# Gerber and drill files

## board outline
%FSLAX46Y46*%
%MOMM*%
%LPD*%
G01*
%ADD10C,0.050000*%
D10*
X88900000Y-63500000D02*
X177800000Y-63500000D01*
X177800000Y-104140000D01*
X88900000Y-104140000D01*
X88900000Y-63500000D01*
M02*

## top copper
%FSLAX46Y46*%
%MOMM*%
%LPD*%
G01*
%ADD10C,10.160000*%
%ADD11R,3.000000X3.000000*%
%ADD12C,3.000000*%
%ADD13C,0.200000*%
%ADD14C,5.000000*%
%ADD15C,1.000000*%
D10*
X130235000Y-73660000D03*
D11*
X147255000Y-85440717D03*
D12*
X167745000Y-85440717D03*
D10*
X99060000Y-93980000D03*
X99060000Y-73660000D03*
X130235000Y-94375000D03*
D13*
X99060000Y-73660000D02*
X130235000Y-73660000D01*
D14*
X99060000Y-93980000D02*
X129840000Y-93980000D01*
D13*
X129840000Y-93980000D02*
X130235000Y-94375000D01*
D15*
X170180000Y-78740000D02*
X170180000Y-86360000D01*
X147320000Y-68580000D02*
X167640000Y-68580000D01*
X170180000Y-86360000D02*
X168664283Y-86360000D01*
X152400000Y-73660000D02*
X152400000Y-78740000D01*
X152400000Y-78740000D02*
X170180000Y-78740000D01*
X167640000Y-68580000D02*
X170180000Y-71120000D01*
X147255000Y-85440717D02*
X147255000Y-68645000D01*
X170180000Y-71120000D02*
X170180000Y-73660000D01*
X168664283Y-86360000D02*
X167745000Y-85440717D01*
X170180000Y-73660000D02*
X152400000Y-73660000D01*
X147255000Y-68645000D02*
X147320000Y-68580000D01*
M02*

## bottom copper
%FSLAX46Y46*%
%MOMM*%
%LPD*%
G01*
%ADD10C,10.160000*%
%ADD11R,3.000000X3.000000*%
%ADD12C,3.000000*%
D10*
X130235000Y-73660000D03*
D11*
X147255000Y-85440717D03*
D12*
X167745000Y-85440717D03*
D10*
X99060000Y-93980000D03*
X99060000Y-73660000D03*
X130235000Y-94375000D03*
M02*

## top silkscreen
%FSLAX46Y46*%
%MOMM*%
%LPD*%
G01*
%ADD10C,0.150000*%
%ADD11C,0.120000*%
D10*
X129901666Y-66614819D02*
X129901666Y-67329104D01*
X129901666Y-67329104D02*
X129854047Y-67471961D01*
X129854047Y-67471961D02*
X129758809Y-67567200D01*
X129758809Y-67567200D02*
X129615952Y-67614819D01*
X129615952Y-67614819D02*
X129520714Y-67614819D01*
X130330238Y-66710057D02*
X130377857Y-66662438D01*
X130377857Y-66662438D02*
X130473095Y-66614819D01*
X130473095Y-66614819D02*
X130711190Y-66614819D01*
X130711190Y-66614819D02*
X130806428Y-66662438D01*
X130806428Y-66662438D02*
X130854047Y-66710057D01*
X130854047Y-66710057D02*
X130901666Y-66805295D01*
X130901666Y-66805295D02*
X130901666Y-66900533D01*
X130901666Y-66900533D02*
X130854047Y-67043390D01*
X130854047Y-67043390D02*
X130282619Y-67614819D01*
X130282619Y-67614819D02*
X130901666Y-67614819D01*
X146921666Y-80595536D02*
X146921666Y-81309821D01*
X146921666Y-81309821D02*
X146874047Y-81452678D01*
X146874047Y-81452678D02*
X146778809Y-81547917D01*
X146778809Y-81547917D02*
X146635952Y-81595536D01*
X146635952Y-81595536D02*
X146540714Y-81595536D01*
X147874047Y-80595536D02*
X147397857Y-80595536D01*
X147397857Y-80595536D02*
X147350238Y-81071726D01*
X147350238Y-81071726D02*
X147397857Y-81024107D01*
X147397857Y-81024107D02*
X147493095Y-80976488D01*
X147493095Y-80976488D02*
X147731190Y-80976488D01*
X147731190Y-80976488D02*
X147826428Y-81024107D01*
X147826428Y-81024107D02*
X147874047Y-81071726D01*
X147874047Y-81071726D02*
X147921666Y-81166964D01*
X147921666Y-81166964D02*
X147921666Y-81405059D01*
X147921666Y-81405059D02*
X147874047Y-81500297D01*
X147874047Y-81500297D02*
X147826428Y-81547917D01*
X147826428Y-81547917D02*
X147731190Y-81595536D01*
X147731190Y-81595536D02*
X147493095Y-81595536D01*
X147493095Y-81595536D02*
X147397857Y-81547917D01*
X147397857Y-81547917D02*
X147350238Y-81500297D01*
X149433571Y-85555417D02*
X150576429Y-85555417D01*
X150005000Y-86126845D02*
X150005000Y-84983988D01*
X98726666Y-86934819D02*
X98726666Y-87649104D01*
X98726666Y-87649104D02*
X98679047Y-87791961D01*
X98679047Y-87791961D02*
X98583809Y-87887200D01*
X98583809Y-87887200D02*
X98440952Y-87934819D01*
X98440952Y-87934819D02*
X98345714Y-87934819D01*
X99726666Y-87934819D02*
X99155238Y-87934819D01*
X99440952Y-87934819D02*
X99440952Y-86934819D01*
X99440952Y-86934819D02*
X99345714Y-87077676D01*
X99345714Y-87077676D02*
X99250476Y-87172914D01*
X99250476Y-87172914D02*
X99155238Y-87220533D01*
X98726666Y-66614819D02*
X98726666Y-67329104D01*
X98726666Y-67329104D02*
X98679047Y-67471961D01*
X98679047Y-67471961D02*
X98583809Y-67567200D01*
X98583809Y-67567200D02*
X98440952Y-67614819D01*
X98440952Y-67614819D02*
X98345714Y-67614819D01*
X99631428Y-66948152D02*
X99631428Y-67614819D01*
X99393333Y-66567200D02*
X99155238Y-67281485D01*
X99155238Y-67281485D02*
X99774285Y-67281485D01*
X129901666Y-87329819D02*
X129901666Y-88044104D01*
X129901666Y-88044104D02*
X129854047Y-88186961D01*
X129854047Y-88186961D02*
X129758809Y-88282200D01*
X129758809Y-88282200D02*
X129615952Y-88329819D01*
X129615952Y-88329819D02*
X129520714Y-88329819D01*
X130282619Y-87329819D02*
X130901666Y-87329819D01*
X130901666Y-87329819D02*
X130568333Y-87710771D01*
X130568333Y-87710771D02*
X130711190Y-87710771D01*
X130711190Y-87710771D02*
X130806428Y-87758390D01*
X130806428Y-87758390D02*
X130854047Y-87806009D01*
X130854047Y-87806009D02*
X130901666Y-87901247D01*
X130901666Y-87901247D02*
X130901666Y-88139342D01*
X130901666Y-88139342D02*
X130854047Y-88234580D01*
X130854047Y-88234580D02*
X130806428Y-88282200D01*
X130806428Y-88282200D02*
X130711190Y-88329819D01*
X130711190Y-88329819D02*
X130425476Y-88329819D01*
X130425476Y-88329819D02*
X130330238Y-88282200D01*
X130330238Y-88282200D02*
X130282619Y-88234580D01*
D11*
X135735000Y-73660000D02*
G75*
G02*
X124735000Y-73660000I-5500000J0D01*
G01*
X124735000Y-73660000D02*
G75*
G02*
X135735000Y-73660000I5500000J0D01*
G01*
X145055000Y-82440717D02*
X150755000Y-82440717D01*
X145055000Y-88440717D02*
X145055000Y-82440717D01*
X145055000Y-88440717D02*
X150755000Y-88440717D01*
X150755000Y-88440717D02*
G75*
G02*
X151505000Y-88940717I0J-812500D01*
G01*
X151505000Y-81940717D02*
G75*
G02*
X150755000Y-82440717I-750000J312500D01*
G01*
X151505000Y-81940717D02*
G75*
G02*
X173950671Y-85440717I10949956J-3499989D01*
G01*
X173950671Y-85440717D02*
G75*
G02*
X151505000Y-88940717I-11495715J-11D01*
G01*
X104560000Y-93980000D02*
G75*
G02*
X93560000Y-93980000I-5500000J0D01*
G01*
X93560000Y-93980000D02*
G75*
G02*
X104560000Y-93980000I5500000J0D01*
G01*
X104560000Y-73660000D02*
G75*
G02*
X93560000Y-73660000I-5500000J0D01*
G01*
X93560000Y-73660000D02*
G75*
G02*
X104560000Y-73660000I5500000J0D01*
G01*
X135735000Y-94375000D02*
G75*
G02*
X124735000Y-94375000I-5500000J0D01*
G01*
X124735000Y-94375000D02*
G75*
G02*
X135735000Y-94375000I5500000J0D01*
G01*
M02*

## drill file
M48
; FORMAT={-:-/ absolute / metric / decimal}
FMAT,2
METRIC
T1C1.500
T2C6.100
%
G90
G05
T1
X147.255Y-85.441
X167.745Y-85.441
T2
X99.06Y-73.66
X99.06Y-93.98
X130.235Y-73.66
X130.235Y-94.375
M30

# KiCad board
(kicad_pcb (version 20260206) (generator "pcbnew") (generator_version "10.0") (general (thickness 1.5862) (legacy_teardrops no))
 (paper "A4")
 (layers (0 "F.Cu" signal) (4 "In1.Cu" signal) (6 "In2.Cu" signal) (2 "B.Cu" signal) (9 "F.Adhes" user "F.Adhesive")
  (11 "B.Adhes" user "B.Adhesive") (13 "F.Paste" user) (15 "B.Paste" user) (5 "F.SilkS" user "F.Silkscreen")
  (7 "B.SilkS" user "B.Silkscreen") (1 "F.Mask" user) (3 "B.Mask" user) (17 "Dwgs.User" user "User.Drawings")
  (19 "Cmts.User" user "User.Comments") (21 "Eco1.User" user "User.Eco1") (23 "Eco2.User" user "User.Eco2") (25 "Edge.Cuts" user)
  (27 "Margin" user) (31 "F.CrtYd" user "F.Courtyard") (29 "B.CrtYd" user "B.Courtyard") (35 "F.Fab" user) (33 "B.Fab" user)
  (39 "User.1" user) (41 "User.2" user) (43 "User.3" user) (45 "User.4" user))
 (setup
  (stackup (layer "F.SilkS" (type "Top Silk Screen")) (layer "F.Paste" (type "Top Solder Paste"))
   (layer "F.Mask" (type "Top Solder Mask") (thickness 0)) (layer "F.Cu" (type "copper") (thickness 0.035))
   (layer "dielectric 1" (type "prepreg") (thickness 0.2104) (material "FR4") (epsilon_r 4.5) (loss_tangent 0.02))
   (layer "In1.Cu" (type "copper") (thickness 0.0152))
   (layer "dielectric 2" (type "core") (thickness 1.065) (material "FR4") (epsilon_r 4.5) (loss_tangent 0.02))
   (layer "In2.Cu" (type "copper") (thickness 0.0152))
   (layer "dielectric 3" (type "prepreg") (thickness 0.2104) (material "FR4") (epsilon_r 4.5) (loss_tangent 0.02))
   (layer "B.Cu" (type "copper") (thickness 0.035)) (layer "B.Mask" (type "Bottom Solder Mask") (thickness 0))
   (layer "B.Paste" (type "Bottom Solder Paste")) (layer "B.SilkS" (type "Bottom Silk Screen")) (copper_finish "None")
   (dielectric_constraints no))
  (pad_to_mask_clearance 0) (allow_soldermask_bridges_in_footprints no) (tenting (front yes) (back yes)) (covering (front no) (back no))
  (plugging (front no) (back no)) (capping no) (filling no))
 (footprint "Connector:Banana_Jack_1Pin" (layer "F.Cu") (at 130.235 73.66)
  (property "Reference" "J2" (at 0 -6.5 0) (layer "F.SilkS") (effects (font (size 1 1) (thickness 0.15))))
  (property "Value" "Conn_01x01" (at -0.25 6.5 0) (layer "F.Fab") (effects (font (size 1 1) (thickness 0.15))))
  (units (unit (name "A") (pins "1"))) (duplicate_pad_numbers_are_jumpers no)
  (fp_circle (center 0 0) (end 5.5 0) (stroke (width 0.12) (type solid)) (fill no) (layer "F.SilkS"))
  (pad "1" thru_hole circle (at 0 0) (size 10.16 10.16) (drill 6.1) (layers "*.Cu" "*.Mask") (remove_unused_layers no) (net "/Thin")))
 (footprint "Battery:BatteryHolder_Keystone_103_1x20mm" (layer "F.Cu") (at 147.255 85.440717)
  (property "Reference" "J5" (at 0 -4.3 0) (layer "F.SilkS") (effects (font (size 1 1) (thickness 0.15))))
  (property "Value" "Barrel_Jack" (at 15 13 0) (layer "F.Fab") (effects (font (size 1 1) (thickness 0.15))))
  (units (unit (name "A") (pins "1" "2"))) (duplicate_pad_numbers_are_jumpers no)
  (fp_line (start -2.2 -3) (end 3.5 -3) (stroke (width 0.12) (type solid)) (layer "F.SilkS"))
  (fp_line (start -2.2 3) (end -2.2 -3) (stroke (width 0.12) (type solid)) (layer "F.SilkS"))
  (fp_line (start -2.2 3) (end 3.5 3) (stroke (width 0.12) (type solid)) (layer "F.SilkS"))
  (fp_arc (start 3.5 3) (mid 3.950694 3.136459) (end 4.25 3.5) (stroke (width 0.12) (type solid)) (layer "F.SilkS"))
  (fp_arc (start 4.25 -3.5) (mid 3.950694 -3.136459) (end 3.5 -3) (stroke (width 0.12) (type solid)) (layer "F.SilkS"))
  (fp_arc (start 4.25 -3.5) (mid 16.971103 -11.358466) (end 26.695671 0) (stroke (width 0.12) (type solid)) (layer "F.SilkS"))
  (fp_arc (start 26.695671 0) (mid 16.971103 11.358466) (end 4.25 3.5) (stroke (width 0.12) (type solid)) (layer "F.SilkS"))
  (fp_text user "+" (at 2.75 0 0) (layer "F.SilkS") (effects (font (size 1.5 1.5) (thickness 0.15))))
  (pad "1" thru_hole rect (at 0 0) (size 3 3) (drill 1.5) (layers "*.Cu" "*.Mask") (remove_unused_layers no) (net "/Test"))
  (pad "2" thru_hole circle (at 20.49 0) (size 3 3) (drill 1.5) (layers "*.Cu" "*.Mask") (remove_unused_layers no) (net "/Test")))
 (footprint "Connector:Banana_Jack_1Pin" (layer "F.Cu") (at 99.06 93.98)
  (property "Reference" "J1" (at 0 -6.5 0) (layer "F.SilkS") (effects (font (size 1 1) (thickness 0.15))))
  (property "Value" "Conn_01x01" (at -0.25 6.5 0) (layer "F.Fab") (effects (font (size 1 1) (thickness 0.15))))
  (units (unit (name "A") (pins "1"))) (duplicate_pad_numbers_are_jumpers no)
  (fp_circle (center 0 0) (end 5.5 0) (stroke (width 0.12) (type solid)) (fill no) (layer "F.SilkS"))
  (pad "1" thru_hole circle (at 0 0) (size 10.16 10.16) (drill 6.1) (layers "*.Cu" "*.Mask") (remove_unused_layers no) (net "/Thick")))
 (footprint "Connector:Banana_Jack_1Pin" (layer "F.Cu") (at 99.06 73.66)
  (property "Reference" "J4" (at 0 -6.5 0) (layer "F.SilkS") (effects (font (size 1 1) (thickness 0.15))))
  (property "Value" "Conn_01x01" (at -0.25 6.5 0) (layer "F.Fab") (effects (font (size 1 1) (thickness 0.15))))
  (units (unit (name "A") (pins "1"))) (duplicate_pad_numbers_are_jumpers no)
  (fp_circle (center 0 0) (end 5.5 0) (stroke (width 0.12) (type solid)) (fill no) (layer "F.SilkS"))
  (pad "1" thru_hole circle (at 0 0) (size 10.16 10.16) (drill 6.1) (layers "*.Cu" "*.Mask") (remove_unused_layers no) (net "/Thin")))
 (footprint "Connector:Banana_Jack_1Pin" (layer "F.Cu") (at 130.235 94.375)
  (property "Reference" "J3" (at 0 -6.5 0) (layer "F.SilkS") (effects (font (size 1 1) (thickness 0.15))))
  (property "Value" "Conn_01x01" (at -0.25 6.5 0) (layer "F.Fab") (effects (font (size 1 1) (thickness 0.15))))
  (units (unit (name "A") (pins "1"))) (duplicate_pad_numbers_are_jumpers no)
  (fp_circle (center 0 0) (end 5.5 0) (stroke (width 0.12) (type solid)) (fill no) (layer "F.SilkS"))
  (pad "1" thru_hole circle (at 0 0) (size 10.16 10.16) (drill 6.1) (layers "*.Cu" "*.Mask") (remove_unused_layers no) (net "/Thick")))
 (gr_rect (start 88.9 63.5) (end 177.8 104.14) (stroke (width 0.05) (type solid)) (fill no) (layer "Edge.Cuts"))
 (segment (start 99.06 73.66) (end 130.235 73.66) (width 0.2) (layer "F.Cu") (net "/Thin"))
 (segment (start 99.06 93.98) (end 129.84 93.98) (width 5) (layer "F.Cu") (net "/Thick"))
 (segment (start 129.84 93.98) (end 130.235 94.375) (width 0.2) (layer "F.Cu") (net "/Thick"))
 (segment (start 170.18 78.74) (end 170.18 86.36) (width 1) (layer "F.Cu") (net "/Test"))
 (segment (start 147.32 68.58) (end 167.64 68.58) (width 1) (layer "F.Cu") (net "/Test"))
 (segment (start 170.18 86.36) (end 168.664283 86.36) (width 1) (layer "F.Cu") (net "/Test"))
 (segment (start 152.4 73.66) (end 152.4 78.74) (width 1) (layer "F.Cu") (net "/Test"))
 (segment (start 152.4 78.74) (end 170.18 78.74) (width 1) (layer "F.Cu") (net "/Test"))
 (segment (start 167.64 68.58) (end 170.18 71.12) (width 1) (layer "F.Cu") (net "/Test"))
 (segment (start 147.255 85.440717) (end 147.255 68.645) (width 1) (layer "F.Cu") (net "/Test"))
 (segment (start 170.18 71.12) (end 170.18 73.66) (width 1) (layer "F.Cu") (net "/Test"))
 (segment (start 168.664283 86.36) (end 167.745 85.440717) (width 1) (layer "F.Cu") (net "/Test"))
 (segment (start 170.18 73.66) (end 152.4 73.66) (width 1) (layer "F.Cu") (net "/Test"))
 (segment (start 147.255 68.645) (end 147.32 68.58) (width 1) (layer "F.Cu") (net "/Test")))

